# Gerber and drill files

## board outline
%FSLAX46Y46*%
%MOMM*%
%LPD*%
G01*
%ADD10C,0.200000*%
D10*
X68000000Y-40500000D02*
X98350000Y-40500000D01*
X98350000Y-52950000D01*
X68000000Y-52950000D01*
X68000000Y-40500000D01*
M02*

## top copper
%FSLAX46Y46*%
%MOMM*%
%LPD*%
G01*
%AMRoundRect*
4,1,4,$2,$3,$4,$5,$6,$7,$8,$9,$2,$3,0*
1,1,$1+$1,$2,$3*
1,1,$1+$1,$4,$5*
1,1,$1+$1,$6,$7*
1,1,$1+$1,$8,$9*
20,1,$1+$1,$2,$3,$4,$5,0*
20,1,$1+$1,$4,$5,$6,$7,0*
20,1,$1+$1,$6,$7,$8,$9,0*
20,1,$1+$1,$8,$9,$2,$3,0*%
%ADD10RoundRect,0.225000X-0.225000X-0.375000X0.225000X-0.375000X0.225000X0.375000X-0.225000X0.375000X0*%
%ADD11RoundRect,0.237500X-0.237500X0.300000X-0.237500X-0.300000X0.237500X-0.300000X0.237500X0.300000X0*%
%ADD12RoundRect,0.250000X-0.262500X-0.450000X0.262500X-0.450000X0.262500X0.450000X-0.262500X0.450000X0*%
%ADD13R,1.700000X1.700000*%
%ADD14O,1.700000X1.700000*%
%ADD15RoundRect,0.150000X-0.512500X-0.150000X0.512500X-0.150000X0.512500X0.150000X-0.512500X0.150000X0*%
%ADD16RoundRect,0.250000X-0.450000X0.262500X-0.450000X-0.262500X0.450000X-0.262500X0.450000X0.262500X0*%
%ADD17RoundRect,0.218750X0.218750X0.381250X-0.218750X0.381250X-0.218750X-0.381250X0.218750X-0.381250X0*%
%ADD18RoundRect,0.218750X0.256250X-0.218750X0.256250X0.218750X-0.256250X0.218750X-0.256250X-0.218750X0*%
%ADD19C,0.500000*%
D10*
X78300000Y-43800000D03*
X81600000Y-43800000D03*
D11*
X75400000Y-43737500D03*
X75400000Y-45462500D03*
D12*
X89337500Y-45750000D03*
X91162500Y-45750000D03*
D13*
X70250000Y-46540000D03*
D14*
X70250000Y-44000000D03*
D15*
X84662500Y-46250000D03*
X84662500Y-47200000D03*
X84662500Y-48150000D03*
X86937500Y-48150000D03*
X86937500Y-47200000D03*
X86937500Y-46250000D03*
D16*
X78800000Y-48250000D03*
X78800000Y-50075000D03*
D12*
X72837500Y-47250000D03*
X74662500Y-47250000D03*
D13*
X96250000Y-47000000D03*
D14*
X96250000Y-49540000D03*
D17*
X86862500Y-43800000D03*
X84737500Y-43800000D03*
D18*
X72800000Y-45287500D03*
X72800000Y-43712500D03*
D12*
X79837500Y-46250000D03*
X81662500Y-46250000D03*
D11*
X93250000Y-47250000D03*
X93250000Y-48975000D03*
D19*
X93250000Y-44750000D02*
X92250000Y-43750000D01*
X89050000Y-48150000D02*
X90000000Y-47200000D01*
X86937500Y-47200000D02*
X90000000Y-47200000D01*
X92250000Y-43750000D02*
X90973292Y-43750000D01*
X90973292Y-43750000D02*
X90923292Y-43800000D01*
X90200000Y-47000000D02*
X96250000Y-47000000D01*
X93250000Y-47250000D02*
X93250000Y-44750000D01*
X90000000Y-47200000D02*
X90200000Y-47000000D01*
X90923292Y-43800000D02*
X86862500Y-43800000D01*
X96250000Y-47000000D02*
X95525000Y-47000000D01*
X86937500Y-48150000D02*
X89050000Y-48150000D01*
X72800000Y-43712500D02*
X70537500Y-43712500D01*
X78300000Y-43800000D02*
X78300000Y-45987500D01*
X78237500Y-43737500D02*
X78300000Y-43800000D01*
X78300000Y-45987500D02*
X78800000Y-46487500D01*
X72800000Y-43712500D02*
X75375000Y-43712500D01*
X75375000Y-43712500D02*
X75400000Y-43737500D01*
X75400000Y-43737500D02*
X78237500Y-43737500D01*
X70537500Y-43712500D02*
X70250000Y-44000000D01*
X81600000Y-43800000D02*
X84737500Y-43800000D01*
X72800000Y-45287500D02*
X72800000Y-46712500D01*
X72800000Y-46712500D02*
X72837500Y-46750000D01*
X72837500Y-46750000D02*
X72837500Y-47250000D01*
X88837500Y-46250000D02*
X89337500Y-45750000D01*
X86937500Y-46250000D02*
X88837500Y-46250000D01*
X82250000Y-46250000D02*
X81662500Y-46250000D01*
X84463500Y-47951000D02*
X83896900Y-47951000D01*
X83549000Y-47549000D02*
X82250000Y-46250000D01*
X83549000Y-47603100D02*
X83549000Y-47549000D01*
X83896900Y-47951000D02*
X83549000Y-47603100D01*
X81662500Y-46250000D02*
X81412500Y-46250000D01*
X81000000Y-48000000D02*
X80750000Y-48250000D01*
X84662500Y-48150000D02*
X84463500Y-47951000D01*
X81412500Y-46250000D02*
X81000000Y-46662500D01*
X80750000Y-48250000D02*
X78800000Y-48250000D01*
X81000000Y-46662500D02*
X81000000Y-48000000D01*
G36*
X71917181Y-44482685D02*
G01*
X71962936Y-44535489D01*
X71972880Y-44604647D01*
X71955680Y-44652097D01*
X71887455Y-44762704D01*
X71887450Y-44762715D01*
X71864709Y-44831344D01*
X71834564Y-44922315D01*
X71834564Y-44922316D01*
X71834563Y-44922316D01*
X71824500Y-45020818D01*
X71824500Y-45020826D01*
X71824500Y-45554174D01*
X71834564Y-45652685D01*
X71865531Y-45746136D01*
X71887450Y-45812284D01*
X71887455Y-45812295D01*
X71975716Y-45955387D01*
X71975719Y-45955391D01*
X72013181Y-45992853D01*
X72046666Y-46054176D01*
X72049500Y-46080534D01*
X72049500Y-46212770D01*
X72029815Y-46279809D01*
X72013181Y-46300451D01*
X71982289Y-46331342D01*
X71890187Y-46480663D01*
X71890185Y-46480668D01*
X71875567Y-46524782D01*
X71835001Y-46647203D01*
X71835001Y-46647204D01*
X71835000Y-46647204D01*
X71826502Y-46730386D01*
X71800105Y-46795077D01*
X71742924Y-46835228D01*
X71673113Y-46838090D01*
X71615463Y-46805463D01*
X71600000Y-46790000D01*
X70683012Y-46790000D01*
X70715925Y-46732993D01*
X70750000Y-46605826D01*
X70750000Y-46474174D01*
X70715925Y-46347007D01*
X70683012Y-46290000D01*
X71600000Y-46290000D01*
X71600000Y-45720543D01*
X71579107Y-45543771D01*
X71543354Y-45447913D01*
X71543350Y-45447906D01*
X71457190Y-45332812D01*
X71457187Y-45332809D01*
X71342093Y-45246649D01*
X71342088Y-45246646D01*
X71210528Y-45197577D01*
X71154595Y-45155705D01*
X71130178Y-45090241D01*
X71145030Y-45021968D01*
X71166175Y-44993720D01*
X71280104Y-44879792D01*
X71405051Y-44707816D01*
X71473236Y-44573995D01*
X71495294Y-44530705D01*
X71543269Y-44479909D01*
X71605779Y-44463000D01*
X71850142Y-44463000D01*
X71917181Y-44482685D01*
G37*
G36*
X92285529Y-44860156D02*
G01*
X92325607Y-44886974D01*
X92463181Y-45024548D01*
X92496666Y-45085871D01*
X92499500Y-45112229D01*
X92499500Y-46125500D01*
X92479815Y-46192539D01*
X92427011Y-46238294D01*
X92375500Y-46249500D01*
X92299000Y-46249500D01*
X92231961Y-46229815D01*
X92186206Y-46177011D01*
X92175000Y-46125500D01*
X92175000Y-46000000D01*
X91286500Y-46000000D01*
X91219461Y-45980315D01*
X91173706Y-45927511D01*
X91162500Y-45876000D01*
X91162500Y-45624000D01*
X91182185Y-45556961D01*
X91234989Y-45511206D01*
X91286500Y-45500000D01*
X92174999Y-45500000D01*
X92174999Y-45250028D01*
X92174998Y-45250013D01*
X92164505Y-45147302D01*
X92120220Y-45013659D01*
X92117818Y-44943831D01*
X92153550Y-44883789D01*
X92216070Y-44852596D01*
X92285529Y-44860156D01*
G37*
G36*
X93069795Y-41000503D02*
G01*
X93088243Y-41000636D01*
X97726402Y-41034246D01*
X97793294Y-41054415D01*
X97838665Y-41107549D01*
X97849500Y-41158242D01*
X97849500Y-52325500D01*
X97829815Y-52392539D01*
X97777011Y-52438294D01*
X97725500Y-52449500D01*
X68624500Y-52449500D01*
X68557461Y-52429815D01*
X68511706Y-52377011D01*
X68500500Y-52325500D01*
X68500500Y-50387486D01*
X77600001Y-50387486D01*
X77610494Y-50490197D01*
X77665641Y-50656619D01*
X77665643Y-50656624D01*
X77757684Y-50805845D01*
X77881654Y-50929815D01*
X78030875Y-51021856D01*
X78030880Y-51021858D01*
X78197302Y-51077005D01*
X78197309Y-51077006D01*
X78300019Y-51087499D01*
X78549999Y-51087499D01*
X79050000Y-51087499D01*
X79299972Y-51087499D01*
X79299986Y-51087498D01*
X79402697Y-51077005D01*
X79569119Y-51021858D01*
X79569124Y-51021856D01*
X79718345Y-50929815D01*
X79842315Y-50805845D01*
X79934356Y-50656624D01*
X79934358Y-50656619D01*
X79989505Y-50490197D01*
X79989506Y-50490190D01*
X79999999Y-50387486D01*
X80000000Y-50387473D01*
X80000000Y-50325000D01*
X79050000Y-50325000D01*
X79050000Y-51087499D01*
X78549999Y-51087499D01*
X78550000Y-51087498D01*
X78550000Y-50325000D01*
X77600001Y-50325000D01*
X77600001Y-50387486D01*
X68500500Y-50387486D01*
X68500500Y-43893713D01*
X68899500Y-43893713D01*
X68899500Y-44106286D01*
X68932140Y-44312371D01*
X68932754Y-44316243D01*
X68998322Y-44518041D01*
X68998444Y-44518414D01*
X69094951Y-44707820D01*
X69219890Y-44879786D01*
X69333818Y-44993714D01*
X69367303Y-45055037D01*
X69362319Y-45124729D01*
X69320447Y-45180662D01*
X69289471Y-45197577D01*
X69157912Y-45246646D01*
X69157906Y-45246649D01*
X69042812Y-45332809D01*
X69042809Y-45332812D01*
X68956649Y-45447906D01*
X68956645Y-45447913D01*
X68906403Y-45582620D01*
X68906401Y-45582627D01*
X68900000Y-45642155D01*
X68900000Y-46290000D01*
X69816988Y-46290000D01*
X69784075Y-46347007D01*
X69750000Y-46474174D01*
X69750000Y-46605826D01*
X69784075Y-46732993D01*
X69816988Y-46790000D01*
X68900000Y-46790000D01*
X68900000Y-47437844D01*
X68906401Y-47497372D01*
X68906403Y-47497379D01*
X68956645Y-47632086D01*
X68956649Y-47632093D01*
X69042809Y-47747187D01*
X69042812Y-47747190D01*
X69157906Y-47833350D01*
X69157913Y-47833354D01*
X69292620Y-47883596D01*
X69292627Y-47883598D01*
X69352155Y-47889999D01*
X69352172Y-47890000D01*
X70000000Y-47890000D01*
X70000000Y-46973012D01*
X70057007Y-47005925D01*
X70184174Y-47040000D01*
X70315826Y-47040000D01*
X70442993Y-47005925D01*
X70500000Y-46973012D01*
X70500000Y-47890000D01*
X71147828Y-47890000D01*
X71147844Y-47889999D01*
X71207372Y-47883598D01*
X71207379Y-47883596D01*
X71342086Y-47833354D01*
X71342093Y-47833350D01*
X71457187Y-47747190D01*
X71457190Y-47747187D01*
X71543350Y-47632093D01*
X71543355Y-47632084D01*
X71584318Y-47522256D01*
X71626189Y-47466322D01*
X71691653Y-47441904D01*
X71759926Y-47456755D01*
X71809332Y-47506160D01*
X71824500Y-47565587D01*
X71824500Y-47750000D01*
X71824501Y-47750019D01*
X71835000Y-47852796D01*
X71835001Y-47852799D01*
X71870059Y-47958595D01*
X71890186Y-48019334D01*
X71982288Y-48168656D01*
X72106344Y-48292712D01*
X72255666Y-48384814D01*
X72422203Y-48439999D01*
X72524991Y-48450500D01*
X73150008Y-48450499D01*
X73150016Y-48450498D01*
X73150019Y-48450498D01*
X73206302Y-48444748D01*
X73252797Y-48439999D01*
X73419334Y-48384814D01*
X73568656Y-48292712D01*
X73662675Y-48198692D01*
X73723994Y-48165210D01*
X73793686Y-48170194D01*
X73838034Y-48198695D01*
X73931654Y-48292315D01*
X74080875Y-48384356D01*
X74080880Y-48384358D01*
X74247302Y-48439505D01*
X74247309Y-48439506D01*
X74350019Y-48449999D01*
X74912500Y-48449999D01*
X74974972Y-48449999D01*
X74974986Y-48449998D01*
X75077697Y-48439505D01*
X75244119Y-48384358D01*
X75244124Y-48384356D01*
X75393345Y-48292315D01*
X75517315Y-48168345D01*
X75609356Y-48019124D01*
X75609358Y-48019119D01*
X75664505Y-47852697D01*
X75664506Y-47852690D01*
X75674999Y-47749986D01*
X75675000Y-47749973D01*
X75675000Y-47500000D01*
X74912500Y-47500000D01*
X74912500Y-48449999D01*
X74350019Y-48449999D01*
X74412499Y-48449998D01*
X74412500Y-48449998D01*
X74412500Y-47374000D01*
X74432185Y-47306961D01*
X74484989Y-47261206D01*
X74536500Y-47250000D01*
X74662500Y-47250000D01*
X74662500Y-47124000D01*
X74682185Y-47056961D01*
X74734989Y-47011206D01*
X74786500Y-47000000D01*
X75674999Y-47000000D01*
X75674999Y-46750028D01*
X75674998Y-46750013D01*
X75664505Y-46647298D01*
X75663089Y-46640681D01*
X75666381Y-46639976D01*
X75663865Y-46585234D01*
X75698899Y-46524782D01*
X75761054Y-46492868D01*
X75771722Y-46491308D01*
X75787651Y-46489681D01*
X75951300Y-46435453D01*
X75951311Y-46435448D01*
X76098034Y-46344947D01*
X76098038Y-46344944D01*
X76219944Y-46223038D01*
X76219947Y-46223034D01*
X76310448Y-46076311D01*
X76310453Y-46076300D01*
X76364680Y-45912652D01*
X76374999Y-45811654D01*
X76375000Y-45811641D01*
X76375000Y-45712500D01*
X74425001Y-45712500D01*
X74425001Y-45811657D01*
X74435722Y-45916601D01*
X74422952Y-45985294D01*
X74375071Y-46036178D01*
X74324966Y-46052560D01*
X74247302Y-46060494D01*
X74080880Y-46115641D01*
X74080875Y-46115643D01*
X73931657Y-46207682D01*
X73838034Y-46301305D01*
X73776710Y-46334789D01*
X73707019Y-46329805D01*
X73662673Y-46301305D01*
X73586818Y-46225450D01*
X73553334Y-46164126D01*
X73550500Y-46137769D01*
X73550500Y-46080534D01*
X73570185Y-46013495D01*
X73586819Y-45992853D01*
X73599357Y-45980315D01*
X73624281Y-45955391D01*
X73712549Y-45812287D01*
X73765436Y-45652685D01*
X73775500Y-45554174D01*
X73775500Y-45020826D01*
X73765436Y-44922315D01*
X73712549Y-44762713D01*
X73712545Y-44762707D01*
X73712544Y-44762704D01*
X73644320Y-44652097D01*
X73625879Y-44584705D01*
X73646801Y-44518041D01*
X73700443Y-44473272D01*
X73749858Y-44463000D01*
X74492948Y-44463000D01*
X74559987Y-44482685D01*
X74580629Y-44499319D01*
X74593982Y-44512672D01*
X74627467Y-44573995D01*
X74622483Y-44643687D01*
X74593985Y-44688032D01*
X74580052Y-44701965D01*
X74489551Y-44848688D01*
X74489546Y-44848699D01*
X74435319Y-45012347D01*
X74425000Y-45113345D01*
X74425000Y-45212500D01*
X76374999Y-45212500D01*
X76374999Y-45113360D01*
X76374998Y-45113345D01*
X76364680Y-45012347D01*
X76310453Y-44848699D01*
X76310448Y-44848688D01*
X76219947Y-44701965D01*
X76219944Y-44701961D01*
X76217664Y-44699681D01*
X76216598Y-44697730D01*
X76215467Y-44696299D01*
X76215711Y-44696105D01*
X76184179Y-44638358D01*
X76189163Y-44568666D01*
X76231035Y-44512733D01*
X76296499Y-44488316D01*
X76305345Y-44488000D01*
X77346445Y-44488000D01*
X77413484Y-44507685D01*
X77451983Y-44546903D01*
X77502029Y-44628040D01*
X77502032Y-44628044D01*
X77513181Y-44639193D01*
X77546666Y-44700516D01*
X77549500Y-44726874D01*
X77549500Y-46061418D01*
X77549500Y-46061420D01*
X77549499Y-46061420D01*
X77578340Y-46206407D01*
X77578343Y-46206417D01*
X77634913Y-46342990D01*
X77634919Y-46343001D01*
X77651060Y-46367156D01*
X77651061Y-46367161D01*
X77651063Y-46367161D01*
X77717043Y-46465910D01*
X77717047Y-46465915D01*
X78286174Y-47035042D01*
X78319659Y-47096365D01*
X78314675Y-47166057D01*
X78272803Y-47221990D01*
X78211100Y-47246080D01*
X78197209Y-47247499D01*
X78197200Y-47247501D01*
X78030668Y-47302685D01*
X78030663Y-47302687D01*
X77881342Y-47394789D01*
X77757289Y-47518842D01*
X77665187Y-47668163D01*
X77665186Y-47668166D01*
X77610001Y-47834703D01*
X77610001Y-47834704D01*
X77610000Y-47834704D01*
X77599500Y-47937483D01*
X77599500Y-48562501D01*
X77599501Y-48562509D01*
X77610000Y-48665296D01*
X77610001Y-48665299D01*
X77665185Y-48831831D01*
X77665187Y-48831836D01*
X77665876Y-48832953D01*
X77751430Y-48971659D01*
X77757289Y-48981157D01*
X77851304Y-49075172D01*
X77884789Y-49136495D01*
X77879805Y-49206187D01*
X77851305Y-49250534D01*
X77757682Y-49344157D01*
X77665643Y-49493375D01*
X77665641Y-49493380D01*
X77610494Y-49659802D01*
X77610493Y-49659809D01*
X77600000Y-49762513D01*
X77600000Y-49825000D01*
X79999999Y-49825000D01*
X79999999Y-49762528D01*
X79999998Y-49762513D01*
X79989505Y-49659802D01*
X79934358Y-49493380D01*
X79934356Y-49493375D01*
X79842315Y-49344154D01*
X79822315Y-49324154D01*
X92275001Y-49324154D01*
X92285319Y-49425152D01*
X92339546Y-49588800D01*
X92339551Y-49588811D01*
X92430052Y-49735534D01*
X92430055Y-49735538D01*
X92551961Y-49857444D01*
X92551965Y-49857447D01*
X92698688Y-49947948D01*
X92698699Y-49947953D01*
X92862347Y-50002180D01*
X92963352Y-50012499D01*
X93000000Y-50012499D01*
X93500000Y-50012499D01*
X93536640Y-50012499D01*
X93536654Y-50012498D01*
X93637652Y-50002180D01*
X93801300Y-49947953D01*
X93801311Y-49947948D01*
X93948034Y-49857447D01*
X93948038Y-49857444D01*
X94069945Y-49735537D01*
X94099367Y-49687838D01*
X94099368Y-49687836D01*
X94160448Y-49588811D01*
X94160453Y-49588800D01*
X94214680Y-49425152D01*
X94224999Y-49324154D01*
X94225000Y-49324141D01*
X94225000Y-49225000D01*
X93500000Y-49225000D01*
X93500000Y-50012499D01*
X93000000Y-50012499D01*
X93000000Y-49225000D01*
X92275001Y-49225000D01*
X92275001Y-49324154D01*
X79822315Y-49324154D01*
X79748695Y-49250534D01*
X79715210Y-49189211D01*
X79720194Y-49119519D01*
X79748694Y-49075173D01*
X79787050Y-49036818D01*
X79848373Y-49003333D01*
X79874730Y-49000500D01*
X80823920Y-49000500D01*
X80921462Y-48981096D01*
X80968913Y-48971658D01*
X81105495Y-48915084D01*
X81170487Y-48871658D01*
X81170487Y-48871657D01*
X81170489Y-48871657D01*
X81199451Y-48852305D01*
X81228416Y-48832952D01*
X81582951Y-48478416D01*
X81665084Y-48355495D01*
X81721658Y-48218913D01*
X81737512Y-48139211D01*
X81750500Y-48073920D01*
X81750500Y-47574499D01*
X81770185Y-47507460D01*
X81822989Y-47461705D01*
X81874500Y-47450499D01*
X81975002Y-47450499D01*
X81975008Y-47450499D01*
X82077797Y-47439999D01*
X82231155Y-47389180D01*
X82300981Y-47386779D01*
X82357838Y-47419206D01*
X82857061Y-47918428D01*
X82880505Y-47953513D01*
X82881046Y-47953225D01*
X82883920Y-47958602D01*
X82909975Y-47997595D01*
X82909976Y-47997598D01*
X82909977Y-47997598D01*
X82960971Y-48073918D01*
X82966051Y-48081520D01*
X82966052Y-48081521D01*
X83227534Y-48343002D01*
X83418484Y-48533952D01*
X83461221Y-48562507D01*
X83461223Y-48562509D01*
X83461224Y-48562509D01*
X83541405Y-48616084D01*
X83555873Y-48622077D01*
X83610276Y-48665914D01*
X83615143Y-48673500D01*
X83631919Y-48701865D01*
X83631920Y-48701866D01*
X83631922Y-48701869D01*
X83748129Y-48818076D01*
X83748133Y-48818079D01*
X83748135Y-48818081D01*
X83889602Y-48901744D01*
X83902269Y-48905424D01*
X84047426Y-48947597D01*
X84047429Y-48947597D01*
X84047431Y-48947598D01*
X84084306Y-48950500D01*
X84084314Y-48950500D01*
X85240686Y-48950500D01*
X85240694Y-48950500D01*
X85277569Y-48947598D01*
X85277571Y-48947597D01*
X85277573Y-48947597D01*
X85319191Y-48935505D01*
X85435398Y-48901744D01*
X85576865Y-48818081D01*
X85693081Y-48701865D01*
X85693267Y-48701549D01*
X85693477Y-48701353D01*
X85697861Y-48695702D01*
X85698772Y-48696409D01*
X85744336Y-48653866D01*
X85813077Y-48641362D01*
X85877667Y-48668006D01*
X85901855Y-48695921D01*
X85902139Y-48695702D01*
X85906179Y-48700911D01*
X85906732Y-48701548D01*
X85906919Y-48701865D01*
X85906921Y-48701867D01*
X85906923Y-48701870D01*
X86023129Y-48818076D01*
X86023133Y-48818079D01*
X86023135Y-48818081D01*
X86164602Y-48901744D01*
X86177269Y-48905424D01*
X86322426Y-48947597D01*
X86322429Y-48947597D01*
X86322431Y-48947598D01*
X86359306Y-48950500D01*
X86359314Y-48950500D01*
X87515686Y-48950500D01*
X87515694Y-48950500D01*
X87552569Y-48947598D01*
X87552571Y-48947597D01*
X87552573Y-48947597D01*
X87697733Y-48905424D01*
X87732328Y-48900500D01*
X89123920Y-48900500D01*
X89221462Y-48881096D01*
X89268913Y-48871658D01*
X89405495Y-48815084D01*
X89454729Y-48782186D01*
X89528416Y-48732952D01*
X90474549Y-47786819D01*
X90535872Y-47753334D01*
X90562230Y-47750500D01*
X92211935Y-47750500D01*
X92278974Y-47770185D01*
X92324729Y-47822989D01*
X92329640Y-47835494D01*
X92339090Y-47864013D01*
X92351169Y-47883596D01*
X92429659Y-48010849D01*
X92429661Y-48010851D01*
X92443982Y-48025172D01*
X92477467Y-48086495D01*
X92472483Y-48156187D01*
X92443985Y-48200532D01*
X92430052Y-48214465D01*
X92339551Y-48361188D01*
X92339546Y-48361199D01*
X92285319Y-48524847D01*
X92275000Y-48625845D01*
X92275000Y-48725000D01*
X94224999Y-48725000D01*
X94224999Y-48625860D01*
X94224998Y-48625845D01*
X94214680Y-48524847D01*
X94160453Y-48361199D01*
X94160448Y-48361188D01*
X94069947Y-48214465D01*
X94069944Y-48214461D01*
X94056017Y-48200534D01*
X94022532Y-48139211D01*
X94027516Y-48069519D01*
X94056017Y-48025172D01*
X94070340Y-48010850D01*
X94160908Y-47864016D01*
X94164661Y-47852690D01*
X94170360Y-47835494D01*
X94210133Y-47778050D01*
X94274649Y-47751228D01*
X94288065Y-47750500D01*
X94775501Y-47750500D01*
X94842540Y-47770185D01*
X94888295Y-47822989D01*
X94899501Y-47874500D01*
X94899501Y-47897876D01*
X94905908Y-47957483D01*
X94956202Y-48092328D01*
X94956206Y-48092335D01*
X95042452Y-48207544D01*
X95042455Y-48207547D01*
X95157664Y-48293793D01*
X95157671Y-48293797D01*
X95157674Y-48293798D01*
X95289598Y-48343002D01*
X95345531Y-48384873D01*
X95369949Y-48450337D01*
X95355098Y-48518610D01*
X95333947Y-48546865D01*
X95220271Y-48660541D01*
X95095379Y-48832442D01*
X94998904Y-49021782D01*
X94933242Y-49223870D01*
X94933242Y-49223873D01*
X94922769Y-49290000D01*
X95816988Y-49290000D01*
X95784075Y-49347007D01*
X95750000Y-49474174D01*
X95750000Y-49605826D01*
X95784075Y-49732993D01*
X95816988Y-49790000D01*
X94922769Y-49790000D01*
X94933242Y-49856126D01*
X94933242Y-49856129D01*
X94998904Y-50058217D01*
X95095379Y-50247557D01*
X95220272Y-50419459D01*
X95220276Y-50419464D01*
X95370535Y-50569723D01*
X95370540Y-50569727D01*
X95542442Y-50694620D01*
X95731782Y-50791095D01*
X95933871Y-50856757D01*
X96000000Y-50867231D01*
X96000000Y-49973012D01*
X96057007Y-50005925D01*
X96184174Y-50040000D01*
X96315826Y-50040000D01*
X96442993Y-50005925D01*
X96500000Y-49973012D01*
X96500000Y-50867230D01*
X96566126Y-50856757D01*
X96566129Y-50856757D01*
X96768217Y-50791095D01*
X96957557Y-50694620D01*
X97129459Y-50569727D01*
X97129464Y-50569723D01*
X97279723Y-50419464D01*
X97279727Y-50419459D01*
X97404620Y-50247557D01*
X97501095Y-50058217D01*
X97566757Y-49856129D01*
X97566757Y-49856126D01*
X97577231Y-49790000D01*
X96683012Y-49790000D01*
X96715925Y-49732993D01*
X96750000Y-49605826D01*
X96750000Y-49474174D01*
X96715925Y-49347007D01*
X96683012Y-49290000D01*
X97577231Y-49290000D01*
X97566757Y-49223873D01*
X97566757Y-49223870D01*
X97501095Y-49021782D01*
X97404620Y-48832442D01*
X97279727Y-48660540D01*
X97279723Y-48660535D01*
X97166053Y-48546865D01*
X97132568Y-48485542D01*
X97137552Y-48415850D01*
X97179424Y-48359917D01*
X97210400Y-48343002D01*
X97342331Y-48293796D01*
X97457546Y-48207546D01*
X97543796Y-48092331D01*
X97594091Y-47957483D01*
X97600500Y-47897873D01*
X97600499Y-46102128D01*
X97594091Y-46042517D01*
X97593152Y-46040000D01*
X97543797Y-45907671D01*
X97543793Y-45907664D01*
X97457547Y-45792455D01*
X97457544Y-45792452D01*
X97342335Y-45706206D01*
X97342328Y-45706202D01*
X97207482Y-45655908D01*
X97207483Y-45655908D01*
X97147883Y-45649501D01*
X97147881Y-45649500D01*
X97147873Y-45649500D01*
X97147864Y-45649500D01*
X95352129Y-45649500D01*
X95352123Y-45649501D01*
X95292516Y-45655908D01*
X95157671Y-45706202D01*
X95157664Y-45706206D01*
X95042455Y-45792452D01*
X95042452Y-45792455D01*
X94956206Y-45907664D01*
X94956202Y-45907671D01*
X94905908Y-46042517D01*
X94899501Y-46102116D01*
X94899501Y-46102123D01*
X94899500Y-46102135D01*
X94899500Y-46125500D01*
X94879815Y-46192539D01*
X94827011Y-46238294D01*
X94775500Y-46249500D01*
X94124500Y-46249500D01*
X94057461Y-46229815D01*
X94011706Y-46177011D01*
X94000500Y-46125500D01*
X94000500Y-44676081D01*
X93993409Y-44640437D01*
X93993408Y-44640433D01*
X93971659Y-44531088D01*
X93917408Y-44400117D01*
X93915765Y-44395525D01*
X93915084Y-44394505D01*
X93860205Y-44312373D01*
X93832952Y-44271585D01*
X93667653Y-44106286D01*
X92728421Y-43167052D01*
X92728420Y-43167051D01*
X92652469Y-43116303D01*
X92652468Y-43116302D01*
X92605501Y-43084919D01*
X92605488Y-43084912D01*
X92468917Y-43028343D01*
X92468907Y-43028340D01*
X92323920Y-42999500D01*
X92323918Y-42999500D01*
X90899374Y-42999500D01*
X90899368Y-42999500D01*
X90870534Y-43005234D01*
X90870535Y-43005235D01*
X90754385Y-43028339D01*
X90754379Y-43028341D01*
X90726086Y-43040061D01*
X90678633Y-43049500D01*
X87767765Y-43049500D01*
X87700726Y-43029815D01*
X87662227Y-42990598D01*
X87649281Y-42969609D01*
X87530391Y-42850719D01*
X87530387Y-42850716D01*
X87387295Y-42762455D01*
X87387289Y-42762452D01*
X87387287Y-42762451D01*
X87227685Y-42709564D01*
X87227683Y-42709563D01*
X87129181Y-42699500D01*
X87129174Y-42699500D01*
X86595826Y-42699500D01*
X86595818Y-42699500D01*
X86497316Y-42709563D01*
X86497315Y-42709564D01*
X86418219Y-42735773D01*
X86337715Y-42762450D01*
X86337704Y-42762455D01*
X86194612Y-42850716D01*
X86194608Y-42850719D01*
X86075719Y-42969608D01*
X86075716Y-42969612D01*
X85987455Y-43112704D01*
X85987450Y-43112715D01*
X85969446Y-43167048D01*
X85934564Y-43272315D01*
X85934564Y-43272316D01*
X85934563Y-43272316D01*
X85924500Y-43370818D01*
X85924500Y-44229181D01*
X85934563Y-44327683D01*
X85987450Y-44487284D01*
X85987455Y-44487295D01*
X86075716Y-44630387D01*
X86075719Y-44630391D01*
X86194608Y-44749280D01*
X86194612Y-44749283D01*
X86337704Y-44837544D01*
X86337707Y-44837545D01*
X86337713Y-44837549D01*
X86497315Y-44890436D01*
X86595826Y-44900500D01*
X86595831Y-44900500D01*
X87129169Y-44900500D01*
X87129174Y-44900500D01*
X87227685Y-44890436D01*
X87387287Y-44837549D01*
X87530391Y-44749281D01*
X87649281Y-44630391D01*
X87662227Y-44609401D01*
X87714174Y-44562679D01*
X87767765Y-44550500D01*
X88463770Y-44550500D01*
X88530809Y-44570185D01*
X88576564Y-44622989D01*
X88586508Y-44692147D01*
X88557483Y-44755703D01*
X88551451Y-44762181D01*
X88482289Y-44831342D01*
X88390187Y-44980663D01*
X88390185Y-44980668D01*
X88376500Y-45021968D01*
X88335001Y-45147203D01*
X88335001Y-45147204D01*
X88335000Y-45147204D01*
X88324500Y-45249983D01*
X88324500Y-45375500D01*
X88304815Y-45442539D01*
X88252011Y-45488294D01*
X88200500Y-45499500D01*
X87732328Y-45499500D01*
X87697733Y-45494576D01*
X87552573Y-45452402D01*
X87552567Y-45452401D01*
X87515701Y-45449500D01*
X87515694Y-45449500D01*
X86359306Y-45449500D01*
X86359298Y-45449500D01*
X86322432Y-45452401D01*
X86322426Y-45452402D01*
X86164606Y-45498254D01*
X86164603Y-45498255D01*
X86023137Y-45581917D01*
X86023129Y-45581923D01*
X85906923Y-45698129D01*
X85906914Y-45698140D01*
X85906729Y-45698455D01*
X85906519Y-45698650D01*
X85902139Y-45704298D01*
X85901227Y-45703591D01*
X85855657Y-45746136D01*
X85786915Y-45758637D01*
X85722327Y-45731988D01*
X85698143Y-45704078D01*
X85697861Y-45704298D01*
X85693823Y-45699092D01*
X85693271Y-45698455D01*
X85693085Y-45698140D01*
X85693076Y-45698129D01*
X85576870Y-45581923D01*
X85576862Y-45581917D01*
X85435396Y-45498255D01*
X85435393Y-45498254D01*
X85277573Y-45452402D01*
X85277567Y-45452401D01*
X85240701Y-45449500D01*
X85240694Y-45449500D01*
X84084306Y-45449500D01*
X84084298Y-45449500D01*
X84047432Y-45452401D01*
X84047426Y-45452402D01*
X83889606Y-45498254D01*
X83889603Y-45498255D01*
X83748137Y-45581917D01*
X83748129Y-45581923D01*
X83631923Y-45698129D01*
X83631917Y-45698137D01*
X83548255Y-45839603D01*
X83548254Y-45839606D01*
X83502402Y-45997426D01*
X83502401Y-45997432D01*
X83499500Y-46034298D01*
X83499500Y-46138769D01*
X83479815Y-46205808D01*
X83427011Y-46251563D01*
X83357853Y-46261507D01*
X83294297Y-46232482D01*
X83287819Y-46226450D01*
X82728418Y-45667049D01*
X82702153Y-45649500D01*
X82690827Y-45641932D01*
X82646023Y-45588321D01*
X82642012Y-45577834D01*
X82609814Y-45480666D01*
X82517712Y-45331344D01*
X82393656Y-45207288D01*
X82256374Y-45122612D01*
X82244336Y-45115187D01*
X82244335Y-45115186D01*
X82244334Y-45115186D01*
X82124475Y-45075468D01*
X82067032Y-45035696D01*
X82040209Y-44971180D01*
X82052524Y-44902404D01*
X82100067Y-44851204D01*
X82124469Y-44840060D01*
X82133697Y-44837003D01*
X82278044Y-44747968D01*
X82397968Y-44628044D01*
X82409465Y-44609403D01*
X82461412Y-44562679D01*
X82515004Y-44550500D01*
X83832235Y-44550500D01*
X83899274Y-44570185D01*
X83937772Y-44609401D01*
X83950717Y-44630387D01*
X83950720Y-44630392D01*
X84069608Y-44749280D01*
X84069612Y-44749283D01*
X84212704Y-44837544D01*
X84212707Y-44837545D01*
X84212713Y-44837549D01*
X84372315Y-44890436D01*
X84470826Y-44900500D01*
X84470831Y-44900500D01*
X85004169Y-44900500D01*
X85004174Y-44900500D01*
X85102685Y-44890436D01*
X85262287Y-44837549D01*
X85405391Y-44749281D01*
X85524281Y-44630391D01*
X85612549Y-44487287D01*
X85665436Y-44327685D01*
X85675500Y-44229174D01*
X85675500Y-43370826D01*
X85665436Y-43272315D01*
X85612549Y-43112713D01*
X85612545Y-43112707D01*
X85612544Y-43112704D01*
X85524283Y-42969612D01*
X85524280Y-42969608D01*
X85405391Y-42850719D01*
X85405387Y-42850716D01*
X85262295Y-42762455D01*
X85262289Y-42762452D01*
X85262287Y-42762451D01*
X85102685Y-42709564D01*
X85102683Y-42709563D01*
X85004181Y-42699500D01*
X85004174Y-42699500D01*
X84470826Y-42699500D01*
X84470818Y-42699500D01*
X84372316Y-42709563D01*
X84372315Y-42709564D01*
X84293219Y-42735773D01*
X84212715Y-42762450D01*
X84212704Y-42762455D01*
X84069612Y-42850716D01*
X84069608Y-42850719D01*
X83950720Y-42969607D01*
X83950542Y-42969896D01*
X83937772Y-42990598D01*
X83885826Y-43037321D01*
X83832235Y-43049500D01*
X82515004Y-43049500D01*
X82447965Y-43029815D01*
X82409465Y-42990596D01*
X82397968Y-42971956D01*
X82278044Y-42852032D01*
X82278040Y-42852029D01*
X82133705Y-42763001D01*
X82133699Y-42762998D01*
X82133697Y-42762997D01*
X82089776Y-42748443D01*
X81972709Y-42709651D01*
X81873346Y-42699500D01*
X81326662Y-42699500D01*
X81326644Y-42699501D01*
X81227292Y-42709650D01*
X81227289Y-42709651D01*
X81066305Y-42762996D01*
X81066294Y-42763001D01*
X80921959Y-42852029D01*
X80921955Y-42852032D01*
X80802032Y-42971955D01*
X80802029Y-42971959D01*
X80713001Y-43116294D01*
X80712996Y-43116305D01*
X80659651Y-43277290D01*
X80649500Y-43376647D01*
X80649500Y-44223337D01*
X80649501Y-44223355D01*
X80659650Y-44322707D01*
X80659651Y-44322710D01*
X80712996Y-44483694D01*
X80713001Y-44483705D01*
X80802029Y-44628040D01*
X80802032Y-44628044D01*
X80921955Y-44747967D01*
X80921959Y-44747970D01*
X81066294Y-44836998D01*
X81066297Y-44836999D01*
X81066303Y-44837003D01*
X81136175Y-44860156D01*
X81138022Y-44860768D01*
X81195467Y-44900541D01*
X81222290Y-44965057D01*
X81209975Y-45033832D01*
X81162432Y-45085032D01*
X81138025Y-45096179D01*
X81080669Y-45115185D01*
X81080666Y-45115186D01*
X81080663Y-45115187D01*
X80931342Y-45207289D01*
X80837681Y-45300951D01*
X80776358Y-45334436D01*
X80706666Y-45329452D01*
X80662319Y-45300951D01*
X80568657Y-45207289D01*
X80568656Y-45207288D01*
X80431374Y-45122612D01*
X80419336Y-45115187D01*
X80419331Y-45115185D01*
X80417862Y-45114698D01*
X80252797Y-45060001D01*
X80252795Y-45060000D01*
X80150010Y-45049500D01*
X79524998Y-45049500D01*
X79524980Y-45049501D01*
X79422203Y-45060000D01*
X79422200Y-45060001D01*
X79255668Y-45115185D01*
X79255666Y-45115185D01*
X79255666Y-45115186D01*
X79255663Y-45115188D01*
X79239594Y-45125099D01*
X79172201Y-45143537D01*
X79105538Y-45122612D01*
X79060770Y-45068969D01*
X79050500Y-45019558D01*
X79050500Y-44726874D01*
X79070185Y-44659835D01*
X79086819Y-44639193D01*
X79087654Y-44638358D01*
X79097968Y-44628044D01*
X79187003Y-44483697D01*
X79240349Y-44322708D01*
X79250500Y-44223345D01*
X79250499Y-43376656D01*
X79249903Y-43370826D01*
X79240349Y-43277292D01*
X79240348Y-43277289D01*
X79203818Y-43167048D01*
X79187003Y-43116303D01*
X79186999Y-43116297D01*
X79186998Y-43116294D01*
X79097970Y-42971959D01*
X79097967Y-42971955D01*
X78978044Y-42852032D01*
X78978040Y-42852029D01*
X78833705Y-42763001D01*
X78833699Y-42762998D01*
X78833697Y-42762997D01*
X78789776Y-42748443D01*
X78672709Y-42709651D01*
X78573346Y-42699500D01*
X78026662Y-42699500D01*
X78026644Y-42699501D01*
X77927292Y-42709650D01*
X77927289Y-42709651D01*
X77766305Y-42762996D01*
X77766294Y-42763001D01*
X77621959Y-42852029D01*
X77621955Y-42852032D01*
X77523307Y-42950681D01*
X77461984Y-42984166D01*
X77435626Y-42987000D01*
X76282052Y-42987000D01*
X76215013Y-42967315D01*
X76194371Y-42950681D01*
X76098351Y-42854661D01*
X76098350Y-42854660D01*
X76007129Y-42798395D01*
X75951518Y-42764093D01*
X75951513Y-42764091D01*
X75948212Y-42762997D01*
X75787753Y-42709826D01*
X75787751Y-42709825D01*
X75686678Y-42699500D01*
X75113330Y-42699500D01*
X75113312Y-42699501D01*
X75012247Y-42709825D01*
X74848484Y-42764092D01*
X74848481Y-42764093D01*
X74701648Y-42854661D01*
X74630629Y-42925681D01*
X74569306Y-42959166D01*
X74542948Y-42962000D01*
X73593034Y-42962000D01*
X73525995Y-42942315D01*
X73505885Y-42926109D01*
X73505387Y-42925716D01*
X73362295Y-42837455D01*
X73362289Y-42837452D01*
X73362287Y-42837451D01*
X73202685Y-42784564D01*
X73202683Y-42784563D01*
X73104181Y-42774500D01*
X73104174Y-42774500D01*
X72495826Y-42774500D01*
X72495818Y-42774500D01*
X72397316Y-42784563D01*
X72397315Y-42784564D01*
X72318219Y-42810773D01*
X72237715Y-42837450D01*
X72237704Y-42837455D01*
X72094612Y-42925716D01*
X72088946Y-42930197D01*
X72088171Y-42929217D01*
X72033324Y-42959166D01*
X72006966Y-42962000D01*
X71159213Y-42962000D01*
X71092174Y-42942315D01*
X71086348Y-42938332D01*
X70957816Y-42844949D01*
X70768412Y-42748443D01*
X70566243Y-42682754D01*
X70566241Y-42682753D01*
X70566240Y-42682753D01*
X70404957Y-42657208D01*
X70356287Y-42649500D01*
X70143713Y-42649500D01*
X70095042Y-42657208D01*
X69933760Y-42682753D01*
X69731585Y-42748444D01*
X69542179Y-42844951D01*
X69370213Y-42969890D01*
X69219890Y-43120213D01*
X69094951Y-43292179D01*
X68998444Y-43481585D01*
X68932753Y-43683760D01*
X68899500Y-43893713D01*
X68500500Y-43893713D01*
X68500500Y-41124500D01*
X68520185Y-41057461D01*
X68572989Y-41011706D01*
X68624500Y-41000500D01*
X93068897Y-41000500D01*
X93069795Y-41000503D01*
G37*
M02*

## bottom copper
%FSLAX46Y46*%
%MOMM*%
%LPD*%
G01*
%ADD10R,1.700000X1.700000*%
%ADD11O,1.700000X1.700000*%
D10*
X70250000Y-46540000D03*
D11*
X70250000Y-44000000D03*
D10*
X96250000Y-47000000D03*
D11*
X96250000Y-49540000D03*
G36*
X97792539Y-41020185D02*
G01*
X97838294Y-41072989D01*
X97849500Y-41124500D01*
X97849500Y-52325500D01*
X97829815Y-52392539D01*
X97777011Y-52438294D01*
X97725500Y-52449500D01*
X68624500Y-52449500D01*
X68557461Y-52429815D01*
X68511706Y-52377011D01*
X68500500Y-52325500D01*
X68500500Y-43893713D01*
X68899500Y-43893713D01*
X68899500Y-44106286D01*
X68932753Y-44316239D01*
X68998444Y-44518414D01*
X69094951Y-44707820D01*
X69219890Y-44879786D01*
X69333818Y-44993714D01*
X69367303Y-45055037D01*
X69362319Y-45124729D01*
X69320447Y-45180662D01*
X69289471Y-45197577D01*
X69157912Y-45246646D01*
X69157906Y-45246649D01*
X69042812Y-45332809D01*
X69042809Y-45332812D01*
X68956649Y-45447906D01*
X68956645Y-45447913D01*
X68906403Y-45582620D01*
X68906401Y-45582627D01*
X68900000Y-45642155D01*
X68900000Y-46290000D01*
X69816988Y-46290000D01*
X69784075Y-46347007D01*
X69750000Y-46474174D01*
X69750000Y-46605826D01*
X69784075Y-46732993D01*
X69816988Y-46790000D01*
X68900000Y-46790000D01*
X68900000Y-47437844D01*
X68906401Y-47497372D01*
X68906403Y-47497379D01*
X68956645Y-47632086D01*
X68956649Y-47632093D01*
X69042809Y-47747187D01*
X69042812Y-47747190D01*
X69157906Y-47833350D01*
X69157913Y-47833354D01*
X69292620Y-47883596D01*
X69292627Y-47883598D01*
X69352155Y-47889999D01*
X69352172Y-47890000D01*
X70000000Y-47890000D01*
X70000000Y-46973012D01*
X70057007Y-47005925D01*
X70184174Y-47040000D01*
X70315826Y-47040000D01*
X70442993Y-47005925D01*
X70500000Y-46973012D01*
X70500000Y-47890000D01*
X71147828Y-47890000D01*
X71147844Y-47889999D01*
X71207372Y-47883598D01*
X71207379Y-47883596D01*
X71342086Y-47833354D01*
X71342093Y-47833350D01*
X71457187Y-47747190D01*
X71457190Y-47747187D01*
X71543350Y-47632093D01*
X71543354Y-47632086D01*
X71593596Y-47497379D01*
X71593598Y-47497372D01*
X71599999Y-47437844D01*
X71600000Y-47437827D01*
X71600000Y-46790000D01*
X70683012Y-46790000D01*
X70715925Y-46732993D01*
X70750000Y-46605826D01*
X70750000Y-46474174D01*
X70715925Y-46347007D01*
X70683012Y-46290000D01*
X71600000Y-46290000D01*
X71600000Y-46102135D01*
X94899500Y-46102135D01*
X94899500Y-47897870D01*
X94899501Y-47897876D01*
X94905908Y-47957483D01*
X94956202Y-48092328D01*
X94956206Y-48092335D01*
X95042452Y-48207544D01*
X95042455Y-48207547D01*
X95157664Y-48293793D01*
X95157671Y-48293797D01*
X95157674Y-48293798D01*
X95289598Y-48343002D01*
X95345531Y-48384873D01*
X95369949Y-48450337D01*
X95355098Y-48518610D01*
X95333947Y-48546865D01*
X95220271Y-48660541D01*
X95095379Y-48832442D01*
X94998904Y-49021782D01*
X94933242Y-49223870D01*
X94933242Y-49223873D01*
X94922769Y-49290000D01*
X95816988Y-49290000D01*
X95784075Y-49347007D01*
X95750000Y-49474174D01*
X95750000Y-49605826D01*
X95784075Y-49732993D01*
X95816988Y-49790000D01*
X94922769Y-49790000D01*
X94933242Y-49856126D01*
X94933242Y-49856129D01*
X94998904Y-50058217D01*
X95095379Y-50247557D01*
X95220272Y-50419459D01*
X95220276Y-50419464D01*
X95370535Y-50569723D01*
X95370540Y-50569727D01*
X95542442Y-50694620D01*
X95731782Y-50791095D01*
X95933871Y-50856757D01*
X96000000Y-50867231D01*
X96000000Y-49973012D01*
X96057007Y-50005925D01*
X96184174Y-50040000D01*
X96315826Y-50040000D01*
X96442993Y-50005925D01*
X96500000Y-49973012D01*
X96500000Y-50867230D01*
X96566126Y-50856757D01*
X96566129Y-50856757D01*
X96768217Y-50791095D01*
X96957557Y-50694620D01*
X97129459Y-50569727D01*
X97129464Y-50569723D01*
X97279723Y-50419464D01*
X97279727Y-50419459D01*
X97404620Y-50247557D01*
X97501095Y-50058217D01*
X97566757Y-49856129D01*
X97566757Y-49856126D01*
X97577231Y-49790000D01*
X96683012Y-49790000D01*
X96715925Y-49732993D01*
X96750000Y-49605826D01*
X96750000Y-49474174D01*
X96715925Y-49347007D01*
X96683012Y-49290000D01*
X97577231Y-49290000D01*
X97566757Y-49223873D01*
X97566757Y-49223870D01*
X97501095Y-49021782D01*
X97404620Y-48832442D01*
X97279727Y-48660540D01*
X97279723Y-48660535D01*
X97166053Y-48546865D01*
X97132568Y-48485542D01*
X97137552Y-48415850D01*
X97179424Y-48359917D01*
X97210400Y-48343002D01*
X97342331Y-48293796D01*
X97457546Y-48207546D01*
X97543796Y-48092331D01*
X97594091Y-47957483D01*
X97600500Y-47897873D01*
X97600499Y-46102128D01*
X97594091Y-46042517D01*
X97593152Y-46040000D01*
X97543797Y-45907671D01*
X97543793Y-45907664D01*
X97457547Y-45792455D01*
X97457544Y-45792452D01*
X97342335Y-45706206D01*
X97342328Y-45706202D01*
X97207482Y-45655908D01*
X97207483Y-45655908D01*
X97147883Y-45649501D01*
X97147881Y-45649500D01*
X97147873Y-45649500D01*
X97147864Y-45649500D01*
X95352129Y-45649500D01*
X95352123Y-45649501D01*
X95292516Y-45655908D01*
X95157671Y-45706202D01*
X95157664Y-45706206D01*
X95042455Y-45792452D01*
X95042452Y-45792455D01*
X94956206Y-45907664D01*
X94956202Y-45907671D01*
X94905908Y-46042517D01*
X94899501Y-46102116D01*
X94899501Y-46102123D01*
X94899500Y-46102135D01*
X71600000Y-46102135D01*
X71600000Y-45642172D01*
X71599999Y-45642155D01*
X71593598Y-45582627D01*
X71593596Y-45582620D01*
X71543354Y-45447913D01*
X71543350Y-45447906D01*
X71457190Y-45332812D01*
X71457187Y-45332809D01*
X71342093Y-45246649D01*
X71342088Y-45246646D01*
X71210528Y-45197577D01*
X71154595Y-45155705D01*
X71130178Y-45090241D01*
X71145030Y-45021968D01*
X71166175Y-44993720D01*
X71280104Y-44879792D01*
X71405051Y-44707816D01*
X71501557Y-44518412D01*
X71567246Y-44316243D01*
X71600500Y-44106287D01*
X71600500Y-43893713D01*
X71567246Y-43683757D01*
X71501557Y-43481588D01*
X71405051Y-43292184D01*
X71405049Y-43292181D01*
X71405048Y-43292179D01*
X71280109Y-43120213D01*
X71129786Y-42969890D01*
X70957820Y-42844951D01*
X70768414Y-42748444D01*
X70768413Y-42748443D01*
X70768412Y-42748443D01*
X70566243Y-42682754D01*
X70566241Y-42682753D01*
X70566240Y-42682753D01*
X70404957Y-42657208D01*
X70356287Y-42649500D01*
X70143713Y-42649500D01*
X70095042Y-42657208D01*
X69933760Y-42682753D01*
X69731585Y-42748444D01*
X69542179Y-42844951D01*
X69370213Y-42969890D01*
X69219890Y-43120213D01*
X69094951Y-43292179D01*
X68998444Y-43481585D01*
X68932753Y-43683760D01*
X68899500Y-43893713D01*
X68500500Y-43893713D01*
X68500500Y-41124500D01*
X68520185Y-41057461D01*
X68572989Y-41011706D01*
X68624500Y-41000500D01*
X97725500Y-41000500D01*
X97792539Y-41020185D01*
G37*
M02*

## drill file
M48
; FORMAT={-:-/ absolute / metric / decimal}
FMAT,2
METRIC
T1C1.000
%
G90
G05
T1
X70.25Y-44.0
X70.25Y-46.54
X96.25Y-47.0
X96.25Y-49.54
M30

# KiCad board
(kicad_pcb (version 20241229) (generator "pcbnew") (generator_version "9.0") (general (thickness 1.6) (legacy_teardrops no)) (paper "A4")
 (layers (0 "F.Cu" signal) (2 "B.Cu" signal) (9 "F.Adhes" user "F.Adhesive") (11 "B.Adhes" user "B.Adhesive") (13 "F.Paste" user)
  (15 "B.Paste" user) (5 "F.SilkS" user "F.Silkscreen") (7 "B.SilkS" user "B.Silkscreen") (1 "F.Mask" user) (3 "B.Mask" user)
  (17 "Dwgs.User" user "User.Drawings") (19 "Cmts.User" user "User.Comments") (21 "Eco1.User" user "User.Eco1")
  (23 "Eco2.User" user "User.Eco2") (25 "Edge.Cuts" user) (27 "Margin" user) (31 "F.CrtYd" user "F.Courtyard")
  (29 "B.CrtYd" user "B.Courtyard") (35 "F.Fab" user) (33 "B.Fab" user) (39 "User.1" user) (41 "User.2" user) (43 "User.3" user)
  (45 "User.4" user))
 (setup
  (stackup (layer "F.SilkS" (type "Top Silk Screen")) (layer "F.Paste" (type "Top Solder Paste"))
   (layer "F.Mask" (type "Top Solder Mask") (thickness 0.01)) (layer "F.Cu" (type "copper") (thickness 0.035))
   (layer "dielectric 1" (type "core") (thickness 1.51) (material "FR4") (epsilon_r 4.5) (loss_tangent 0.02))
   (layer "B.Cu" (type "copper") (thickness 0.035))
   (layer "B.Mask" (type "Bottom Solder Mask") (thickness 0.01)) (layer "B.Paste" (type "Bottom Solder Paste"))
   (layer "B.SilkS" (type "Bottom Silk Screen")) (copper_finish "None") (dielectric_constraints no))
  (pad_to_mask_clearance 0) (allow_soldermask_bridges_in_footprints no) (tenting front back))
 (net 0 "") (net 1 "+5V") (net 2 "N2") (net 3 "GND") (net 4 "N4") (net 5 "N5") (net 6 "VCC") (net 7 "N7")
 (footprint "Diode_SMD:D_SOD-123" (layer "F.Cu") (at 79.95 43.8)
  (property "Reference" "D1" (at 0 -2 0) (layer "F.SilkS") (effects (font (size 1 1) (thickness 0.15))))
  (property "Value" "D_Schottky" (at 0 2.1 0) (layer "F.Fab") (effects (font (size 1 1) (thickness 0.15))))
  (pad "1" smd roundrect (at -1.65 0) (size 0.9 1.2) (layers "F.Cu" "F.Mask" "F.Paste") (roundrect_rratio 0.25) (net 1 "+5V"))
  (pad "2" smd roundrect (at 1.65 0) (size 0.9 1.2) (layers "F.Cu" "F.Mask" "F.Paste") (roundrect_rratio 0.25) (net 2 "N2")))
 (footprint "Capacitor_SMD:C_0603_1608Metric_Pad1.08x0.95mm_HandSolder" (layer "F.Cu") (at 75.4 44.6 -90)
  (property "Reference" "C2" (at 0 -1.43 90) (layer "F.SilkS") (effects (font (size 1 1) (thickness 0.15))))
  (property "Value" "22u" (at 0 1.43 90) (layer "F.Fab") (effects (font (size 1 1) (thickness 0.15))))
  (pad "1" smd roundrect (at -0.8625 0 270) (size 1.075 0.95) (layers "F.Cu" "F.Mask" "F.Paste") (roundrect_rratio 0.25) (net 1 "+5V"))
  (pad "2" smd roundrect (at 0.8625 0 270) (size 1.075 0.95) (layers "F.Cu" "F.Mask" "F.Paste") (roundrect_rratio 0.25) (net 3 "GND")))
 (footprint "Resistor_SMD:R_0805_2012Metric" (layer "F.Cu") (at 90.25 45.75)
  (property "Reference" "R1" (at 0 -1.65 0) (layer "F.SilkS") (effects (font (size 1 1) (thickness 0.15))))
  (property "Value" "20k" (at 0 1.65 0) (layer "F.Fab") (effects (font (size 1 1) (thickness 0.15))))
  (pad "1" smd roundrect (at -0.9125 0) (size 1.025 1.4) (layers "F.Cu" "F.Mask" "F.Paste") (roundrect_rratio 0.243902) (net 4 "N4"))
  (pad "2" smd roundrect (at 0.9125 0) (size 1.025 1.4) (layers "F.Cu" "F.Mask" "F.Paste") (roundrect_rratio 0.243902) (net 3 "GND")))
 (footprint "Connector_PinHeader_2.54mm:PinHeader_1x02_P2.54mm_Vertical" (layer "F.Cu") (at 70.25 46.54 180)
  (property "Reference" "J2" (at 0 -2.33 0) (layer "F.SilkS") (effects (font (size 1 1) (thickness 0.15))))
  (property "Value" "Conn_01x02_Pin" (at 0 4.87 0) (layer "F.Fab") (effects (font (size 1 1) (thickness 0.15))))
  (pad "1" thru_hole rect (at 0 0 180) (size 1.7 1.7) (drill 1) (layers "*.Cu" "*.Mask") (remove_unused_layers no) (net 3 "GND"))
  (pad "2" thru_hole oval (at 0 2.54 180) (size 1.7 1.7) (drill 1) (layers "*.Cu" "*.Mask") (remove_unused_layers no) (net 1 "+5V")))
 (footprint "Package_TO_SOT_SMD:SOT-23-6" (layer "F.Cu") (at 85.8 47.2)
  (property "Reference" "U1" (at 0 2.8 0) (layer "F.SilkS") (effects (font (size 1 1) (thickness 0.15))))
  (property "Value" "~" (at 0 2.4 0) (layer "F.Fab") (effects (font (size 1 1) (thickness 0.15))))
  (pad "1" smd roundrect (at -1.1375 -0.95) (size 1.325 0.6) (layers "F.Cu" "F.Mask" "F.Paste") (roundrect_rratio 0.25) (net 2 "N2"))
  (pad "2" smd roundrect (at -1.1375 0) (size 1.325 0.6) (layers "F.Cu" "F.Mask" "F.Paste") (roundrect_rratio 0.25) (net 3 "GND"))
  (pad "3" smd roundrect (at -1.1375 0.95) (size 1.325 0.6) (layers "F.Cu" "F.Mask" "F.Paste") (roundrect_rratio 0.25) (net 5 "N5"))
  (pad "4" smd roundrect (at 1.1375 0.95) (size 1.325 0.6) (layers "F.Cu" "F.Mask" "F.Paste") (roundrect_rratio 0.25) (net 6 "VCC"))
  (pad "5" smd roundrect (at 1.1375 0) (size 1.325 0.6) (layers "F.Cu" "F.Mask" "F.Paste") (roundrect_rratio 0.25) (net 6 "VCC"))
  (pad "6" smd roundrect (at 1.1375 -0.95) (size 1.325 0.6) (layers "F.Cu" "F.Mask" "F.Paste") (roundrect_rratio 0.25) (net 4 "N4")))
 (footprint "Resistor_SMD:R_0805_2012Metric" (layer "F.Cu") (at 78.8 49.1625 -90)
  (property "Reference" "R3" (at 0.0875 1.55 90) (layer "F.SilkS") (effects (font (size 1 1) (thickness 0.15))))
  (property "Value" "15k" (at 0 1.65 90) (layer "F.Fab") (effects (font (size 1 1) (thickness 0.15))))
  (pad "1" smd roundrect (at -0.9125 0 270) (size 1.025 1.4) (layers "F.Cu" "F.Mask" "F.Paste") (roundrect_rratio 0.243902) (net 5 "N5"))
  (pad "2" smd roundrect (at 0.9125 0 270) (size 1.025 1.4) (layers "F.Cu" "F.Mask" "F.Paste") (roundrect_rratio 0.243902) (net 3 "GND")))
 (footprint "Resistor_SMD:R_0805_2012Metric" (layer "F.Cu") (at 73.75 47.25)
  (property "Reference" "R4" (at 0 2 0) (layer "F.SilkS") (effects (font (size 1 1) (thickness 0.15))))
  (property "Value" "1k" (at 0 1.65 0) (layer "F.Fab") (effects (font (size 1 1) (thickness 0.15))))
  (pad "1" smd roundrect (at -0.9125 0) (size 1.025 1.4) (layers "F.Cu" "F.Mask" "F.Paste") (roundrect_rratio 0.243902) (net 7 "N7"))
  (pad "2" smd roundrect (at 0.9125 0) (size 1.025 1.4) (layers "F.Cu" "F.Mask" "F.Paste") (roundrect_rratio 0.243902) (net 3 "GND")))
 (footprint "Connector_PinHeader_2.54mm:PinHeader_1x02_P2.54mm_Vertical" (layer "F.Cu") (at 96.25 47)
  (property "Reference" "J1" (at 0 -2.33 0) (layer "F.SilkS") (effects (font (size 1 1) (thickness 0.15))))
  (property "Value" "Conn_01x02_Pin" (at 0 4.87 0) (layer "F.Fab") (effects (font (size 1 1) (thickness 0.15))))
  (pad "1" thru_hole rect (at 0 0) (size 1.7 1.7) (drill 1) (layers "*.Cu" "*.Mask") (remove_unused_layers no) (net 6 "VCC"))
  (pad "2" thru_hole oval (at 0 2.54) (size 1.7 1.7) (drill 1) (layers "*.Cu" "*.Mask") (remove_unused_layers no) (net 3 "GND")))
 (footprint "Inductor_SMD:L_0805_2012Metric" (layer "F.Cu") (at 85.8 43.8 180)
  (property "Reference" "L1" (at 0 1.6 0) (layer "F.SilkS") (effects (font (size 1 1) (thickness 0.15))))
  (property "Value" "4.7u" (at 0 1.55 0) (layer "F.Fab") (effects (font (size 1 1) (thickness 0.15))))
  (pad "1" smd roundrect (at -1.0625 0 180) (size 0.875 1.2) (layers "F.Cu" "F.Mask" "F.Paste") (roundrect_rratio 0.25) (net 6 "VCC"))
  (pad "2" smd roundrect (at 1.0625 0 180) (size 0.875 1.2) (layers "F.Cu" "F.Mask" "F.Paste") (roundrect_rratio 0.25) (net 2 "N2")))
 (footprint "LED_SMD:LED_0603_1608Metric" (layer "F.Cu") (at 72.8 44.5 90)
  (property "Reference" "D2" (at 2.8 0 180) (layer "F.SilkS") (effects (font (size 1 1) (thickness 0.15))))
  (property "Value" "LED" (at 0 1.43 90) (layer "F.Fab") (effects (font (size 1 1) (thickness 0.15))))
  (pad "1" smd roundrect (at -0.7875 0 90) (size 0.875 0.95) (layers "F.Cu" "F.Mask" "F.Paste") (roundrect_rratio 0.25) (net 7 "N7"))
  (pad "2" smd roundrect (at 0.7875 0 90) (size 0.875 0.95) (layers "F.Cu" "F.Mask" "F.Paste") (roundrect_rratio 0.25) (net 1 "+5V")))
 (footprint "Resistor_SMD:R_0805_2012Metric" (layer "F.Cu") (at 80.75 46.25)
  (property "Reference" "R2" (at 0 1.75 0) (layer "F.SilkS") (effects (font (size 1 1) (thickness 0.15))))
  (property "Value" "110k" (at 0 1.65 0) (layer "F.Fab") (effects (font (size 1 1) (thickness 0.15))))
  (pad "1" smd roundrect (at -0.9125 0) (size 1.025 1.4) (layers "F.Cu" "F.Mask" "F.Paste") (roundrect_rratio 0.243902) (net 1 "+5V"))
  (pad "2" smd roundrect (at 0.9125 0) (size 1.025 1.4) (layers "F.Cu" "F.Mask" "F.Paste") (roundrect_rratio 0.243902) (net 5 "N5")))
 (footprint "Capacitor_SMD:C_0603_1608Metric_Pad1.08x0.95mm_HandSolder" (layer "F.Cu") (at 93.25 48.1125 -90)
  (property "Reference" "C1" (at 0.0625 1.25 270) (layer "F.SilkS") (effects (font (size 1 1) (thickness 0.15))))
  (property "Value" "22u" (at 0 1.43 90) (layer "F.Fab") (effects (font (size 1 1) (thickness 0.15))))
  (pad "1" smd roundrect (at -0.8625 0 270) (size 1.075 0.95) (layers "F.Cu" "F.Mask" "F.Paste") (roundrect_rratio 0.25) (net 6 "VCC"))
  (pad "2" smd roundrect (at 0.8625 0 270) (size 1.075 0.95) (layers "F.Cu" "F.Mask" "F.Paste") (roundrect_rratio 0.25) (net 3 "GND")))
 (gr_rect (start 68 40.5) (end 98.35 52.95) (stroke (width 0.2) (type solid)) (fill no) (layer "Edge.Cuts"))
 (segment (start 93.25 44.75) (end 92.25 43.75) (width 0.5) (layer "F.Cu") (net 6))
 (segment (start 89.05 48.15) (end 90 47.2) (width 0.5) (layer "F.Cu") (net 6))
 (segment (start 86.9375 47.2) (end 90 47.2) (width 0.5) (layer "F.Cu") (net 6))
 (segment (start 92.25 43.75) (end 90.973292 43.75) (width 0.5) (layer "F.Cu") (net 6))
 (segment (start 90.973292 43.75) (end 90.923292 43.8) (width 0.5) (layer "F.Cu") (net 6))
 (segment (start 90.2 47) (end 96.25 47) (width 0.5) (layer "F.Cu") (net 6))
 (segment (start 93.25 47.25) (end 93.25 44.75) (width 0.5) (layer "F.Cu") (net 6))
 (segment (start 90 47.2) (end 90.2 47) (width 0.5) (layer "F.Cu") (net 6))
 (segment (start 90.923292 43.8) (end 86.8625 43.8) (width 0.5) (layer "F.Cu") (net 6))
 (segment (start 96.25 47) (end 95.525 47) (width 0.5) (layer "F.Cu") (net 6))
 (segment (start 86.9375 48.15) (end 89.05 48.15) (width 0.5) (layer "F.Cu") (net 6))
 (segment (start 72.8 43.7125) (end 70.5375 43.7125) (width 0.5) (layer "F.Cu") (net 1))
 (segment (start 78.3 43.8) (end 78.3 45.9875) (width 0.5) (layer "F.Cu") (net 1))
 (segment (start 78.2375 43.7375) (end 78.3 43.8) (width 0.5) (layer "F.Cu") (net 1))
 (segment (start 78.3 45.9875) (end 78.8 46.4875) (width 0.5) (layer "F.Cu") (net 1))
 (segment (start 72.8 43.7125) (end 75.375 43.7125) (width 0.5) (layer "F.Cu") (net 1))
 (segment (start 75.375 43.7125) (end 75.4 43.7375) (width 0.5) (layer "F.Cu") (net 1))
 (segment (start 75.4 43.7375) (end 78.2375 43.7375) (width 0.5) (layer "F.Cu") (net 1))
 (segment (start 70.5375 43.7125) (end 70.25 44) (width 0.5) (layer "F.Cu") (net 1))
 (segment (start 81.6 43.8) (end 84.7375 43.8) (width 0.5) (layer "F.Cu") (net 2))
 (segment (start 72.8 45.2875) (end 72.8 46.7125) (width 0.5) (layer "F.Cu") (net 7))
 (segment (start 72.8 46.7125) (end 72.8375 46.75) (width 0.5) (layer "F.Cu") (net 7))
 (segment (start 72.8375 46.75) (end 72.8375 47.25) (width 0.5) (layer "F.Cu") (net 7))
 (segment (start 88.8375 46.25) (end 89.3375 45.75) (width 0.5) (layer "F.Cu") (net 4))
 (segment (start 86.9375 46.25) (end 88.8375 46.25) (width 0.5) (layer "F.Cu") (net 4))
 (segment (start 82.25 46.25) (end 81.6625 46.25) (width 0.5) (layer "F.Cu") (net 5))
 (segment (start 84.4635 47.951) (end 83.8969 47.951) (width 0.5) (layer "F.Cu") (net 5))
 (segment (start 83.549 47.549) (end 82.25 46.25) (width 0.5) (layer "F.Cu") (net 5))
 (segment (start 83.549 47.6031) (end 83.549 47.549) (width 0.5) (layer "F.Cu") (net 5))
 (segment (start 83.8969 47.951) (end 83.549 47.6031) (width 0.5) (layer "F.Cu") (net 5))
 (segment (start 81.6625 46.25) (end 81.4125 46.25) (width 0.5) (layer "F.Cu") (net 5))
 (segment (start 81 48) (end 80.75 48.25) (width 0.5) (layer "F.Cu") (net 5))
 (segment (start 84.6625 48.15) (end 84.4635 47.951) (width 0.5) (layer "F.Cu") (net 5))
 (segment (start 81.4125 46.25) (end 81 46.6625) (width 0.5) (layer "F.Cu") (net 5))
 (segment (start 80.75 48.25) (end 78.8 48.25) (width 0.5) (layer "F.Cu") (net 5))
 (segment (start 81 46.6625) (end 81 48) (width 0.5) (layer "F.Cu") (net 5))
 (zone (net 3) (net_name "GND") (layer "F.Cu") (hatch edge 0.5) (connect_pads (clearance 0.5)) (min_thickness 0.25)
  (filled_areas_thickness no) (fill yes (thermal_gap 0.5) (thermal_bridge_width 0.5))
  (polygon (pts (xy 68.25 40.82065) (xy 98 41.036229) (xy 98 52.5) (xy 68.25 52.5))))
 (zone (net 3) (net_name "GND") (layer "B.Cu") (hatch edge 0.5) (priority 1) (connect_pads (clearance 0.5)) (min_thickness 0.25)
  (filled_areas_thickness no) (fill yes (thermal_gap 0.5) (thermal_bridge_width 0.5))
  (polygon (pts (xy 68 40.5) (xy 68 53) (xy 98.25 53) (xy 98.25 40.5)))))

